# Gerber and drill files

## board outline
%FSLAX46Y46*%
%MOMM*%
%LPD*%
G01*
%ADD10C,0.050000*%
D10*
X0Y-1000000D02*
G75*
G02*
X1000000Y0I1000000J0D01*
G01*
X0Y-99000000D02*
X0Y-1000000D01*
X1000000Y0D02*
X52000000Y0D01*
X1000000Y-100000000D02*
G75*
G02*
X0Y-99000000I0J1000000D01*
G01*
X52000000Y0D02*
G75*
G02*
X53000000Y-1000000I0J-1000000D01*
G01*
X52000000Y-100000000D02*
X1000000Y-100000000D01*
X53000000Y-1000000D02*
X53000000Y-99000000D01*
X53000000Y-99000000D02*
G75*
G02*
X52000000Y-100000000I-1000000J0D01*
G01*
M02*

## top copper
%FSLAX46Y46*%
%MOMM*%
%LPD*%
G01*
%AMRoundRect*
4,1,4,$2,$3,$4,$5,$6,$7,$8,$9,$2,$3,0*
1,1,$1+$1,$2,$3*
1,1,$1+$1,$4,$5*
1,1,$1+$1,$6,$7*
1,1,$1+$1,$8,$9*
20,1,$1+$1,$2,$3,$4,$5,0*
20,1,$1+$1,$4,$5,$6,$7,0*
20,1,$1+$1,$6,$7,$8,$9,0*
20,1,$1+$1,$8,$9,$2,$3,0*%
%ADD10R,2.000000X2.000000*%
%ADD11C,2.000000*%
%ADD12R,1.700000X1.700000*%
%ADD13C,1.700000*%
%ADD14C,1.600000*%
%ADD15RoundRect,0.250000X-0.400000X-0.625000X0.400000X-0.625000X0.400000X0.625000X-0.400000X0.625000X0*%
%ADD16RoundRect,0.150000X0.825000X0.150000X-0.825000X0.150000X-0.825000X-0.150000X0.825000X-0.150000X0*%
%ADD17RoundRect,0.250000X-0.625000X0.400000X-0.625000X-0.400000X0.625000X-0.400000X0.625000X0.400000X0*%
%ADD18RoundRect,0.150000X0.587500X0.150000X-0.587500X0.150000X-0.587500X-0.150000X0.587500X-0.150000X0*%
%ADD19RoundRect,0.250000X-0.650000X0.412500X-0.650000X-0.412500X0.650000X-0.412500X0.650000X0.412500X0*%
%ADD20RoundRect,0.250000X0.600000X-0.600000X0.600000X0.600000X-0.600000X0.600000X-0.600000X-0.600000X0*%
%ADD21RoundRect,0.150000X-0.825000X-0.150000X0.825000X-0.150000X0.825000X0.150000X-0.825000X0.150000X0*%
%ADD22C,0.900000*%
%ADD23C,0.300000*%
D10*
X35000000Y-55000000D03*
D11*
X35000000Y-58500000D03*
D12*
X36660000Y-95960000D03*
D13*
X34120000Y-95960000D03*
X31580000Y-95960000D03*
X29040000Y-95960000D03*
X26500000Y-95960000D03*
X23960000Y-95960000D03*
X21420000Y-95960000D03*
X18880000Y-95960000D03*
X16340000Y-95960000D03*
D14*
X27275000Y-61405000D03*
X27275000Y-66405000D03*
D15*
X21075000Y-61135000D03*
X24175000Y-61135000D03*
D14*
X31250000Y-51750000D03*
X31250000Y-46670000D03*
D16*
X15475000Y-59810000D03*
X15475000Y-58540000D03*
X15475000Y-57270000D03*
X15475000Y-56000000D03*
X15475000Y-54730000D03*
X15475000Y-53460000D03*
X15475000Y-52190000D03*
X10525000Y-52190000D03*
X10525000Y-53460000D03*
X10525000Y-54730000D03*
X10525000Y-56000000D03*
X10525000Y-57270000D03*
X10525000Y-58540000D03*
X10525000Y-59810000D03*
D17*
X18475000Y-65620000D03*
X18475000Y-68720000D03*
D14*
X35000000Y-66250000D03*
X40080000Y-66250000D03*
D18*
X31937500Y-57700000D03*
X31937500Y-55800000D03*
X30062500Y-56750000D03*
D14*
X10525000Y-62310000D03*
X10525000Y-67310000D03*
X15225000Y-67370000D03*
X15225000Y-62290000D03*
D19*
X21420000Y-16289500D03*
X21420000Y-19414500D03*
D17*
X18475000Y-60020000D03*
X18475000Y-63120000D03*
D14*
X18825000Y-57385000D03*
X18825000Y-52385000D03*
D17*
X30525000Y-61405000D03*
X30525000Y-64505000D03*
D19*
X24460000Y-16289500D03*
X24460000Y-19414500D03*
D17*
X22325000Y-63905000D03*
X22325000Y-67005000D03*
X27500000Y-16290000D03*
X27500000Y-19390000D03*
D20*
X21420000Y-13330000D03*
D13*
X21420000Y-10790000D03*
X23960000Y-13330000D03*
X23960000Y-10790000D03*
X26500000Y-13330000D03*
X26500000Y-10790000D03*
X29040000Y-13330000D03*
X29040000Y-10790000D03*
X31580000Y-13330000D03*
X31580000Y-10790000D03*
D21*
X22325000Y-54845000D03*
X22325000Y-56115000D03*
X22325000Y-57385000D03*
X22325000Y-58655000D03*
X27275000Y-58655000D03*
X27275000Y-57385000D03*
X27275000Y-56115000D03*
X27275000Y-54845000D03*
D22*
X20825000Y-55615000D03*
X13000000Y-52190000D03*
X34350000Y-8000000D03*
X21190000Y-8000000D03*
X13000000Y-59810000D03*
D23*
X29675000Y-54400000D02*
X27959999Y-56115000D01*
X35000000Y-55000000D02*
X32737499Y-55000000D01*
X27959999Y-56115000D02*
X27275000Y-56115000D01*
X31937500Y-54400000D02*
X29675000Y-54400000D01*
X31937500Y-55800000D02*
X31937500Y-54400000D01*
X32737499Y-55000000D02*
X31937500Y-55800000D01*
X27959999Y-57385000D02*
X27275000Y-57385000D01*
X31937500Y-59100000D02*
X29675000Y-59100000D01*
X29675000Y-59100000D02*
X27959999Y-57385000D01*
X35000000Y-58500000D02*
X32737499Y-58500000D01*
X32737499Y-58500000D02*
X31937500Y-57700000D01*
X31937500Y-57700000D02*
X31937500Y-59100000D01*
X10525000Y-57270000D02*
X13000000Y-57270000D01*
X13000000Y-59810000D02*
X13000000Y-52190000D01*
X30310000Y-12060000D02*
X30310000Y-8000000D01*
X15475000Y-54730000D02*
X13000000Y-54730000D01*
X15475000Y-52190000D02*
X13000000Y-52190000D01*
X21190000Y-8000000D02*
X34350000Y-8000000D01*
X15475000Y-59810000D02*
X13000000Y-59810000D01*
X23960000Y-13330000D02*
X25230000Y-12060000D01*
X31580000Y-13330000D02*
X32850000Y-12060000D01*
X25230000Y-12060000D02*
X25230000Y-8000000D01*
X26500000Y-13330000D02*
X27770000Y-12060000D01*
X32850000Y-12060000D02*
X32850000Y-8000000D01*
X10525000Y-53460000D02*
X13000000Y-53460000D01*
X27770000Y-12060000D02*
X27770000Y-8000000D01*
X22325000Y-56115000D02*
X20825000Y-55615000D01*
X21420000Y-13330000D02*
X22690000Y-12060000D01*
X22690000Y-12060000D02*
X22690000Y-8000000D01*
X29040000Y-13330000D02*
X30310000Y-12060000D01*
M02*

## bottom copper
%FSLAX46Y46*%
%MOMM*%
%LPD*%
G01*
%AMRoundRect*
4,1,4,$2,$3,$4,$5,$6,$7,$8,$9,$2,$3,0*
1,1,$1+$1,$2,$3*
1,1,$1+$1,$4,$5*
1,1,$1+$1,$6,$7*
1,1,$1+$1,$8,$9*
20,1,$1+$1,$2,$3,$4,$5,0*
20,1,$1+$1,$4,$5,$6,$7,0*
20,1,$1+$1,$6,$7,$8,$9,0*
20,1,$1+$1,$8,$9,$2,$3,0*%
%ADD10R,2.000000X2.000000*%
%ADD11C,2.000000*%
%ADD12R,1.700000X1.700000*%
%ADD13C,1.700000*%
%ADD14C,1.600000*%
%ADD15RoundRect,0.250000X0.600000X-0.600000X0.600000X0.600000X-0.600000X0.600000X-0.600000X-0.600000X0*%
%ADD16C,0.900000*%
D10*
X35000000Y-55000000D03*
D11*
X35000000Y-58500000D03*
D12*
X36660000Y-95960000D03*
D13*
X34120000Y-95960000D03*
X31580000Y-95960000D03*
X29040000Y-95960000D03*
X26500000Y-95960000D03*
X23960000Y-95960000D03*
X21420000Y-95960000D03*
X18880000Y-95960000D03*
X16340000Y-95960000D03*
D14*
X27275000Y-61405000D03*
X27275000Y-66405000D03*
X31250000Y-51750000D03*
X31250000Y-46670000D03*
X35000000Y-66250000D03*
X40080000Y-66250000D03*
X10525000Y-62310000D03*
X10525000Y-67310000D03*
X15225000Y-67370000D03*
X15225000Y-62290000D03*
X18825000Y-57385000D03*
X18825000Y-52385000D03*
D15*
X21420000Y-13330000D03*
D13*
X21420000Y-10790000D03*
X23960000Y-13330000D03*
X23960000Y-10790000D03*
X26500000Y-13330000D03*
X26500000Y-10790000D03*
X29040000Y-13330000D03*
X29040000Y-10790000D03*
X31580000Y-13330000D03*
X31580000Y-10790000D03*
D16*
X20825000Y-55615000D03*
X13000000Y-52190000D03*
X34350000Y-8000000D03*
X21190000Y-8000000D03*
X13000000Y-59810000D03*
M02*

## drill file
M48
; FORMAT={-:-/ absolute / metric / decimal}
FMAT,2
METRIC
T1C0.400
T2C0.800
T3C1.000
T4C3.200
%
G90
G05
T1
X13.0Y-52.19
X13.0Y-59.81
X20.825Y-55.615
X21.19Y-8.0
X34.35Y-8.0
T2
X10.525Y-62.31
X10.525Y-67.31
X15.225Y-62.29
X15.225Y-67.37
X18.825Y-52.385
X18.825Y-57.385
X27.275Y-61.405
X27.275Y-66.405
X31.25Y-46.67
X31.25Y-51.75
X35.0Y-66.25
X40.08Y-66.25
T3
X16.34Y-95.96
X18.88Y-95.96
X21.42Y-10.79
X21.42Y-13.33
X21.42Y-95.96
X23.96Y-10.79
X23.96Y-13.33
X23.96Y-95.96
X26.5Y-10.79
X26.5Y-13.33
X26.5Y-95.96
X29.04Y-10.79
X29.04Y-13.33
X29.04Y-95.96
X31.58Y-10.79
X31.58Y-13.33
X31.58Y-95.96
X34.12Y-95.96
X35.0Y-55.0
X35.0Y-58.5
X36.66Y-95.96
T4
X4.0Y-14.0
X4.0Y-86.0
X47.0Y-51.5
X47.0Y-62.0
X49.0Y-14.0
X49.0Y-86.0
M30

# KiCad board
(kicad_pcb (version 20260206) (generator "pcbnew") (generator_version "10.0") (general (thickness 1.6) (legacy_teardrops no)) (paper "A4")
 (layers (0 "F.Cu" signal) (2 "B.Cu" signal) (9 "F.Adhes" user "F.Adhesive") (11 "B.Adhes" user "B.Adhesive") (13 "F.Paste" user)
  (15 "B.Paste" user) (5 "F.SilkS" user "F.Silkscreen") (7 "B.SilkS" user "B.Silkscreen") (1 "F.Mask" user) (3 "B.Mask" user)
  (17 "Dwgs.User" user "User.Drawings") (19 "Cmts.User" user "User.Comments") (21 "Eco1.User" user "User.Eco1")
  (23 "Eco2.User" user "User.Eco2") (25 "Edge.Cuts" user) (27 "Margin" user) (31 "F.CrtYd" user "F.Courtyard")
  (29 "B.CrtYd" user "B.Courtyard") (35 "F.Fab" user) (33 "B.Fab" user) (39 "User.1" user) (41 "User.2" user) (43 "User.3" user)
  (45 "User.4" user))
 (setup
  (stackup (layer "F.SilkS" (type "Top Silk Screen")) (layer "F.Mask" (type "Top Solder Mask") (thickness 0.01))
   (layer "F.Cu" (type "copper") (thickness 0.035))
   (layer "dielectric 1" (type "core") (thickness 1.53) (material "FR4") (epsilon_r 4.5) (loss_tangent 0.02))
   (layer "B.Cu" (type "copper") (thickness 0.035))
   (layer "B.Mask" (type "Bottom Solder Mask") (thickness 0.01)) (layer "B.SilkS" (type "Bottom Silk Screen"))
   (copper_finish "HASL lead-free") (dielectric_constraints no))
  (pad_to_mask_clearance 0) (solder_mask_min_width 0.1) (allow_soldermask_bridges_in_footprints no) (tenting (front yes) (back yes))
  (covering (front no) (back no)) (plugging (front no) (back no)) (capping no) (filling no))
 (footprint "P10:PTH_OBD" (layer "F.Cu") (at 35 55 -90)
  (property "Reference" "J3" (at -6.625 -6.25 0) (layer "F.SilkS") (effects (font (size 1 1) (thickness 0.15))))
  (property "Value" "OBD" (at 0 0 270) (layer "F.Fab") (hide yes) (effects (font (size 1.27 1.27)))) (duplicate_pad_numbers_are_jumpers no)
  (pad "" np_thru_hole circle (at -3.5 -12 270) (size 3.2 3.2) (drill 3.2) (layers "*.Cu" "*.Mask"))
  (pad "" np_thru_hole circle (at 7 -12 270) (size 3.2 3.2) (drill 3.2) (layers "*.Cu" "*.Mask"))
  (pad "1" thru_hole rect (at 0 0 270) (size 2 2) (drill 1) (layers "*.Cu" "*.Mask") (remove_unused_layers no) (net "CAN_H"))
  (pad "2" thru_hole circle (at 3.5 0 270) (size 2 2) (drill 1) (layers "*.Cu" "*.Mask") (remove_unused_layers no) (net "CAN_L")))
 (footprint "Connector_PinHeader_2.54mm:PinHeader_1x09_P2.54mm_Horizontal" (layer "F.Cu") (at 36.66 95.96 -90)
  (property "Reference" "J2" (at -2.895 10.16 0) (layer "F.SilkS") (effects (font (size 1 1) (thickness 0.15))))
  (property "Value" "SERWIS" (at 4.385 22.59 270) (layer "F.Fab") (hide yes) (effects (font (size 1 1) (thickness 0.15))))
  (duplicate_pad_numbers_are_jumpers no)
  (pad "1" thru_hole rect (at 0 0 270) (size 1.7 1.7) (drill 1) (layers "*.Cu" "*.Mask") (remove_unused_layers no) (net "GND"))
  (pad "2" thru_hole circle (at 0 2.54 270) (size 1.7 1.7) (drill 1) (layers "*.Cu" "*.Mask") (remove_unused_layers no)
   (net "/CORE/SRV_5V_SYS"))
  (pad "3" thru_hole circle (at 0 5.08 270) (size 1.7 1.7) (drill 1) (layers "*.Cu" "*.Mask") (remove_unused_layers no)
   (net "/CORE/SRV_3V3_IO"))
  (pad "4" thru_hole circle (at 0 7.62 270) (size 1.7 1.7) (drill 1) (layers "*.Cu" "*.Mask") (remove_unused_layers no)
   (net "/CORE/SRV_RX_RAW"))
  (pad "5" thru_hole circle (at 0 10.16 270) (size 1.7 1.7) (drill 1) (layers "*.Cu" "*.Mask") (remove_unused_layers no)
   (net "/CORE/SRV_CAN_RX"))
  (pad "6" thru_hole circle (at 0 12.7 270) (size 1.7 1.7) (drill 1) (layers "*.Cu" "*.Mask") (remove_unused_layers no)
   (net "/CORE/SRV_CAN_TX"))
  (pad "7" thru_hole circle (at 0 15.24 270) (size 1.7 1.7) (drill 1) (layers "*.Cu" "*.Mask") (remove_unused_layers no)
   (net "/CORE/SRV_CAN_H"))
  (pad "8" thru_hole circle (at 0 17.78 270) (size 1.7 1.7) (drill 1) (layers "*.Cu" "*.Mask") (remove_unused_layers no)
   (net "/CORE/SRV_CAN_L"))
  (pad "9" thru_hole circle (at 0 20.32 270) (size 1.7 1.7) (drill 1) (layers "*.Cu" "*.Mask") (remove_unused_layers no) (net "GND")))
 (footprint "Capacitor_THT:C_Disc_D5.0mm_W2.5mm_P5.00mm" (layer "F.Cu") (at 27.275 61.405 -90)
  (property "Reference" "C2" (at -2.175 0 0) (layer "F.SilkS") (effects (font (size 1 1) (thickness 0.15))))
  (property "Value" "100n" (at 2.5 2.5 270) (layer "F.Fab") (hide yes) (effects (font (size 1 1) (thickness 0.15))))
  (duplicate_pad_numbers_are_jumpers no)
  (pad "1" thru_hole circle (at 0 0 270) (size 1.6 1.6) (drill 0.8) (layers "*.Cu" "*.Mask") (remove_unused_layers no) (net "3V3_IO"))
  (pad "2" thru_hole circle (at 5 0 270) (size 1.6 1.6) (drill 0.8) (layers "*.Cu" "*.Mask") (remove_unused_layers no) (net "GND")))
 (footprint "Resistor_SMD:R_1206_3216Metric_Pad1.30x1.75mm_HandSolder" (layer "F.Cu") (at 22.625 61.135)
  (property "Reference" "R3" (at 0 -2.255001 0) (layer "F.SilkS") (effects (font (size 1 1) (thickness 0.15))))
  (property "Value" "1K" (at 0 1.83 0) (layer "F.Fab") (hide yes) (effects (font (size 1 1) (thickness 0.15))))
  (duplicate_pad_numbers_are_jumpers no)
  (pad "1" smd roundrect (at -1.55 0) (size 1.3 1.75) (layers "F.Cu" "F.Mask" "F.Paste") (roundrect_rratio 0.192308) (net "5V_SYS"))
  (pad "2" smd roundrect (at 1.55 0) (size 1.3 1.75) (layers "F.Cu" "F.Mask" "F.Paste") (roundrect_rratio 0.192308) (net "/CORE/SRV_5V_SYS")))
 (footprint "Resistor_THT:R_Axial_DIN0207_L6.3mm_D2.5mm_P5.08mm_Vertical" (layer "F.Cu") (at 31.25 51.75 90)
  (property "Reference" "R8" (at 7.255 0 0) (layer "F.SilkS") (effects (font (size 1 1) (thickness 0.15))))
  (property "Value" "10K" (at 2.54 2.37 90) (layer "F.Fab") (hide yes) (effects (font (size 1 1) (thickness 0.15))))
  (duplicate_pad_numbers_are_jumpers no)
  (pad "1" thru_hole circle (at 0 0 90) (size 1.6 1.6) (drill 0.8) (layers "*.Cu" "*.Mask") (remove_unused_layers no) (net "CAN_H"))
  (pad "2" thru_hole circle (at 5.08 0 90) (size 1.6 1.6) (drill 0.8) (layers "*.Cu" "*.Mask") (remove_unused_layers no)
   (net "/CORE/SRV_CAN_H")))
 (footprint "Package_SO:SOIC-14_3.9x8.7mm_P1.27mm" (layer "F.Cu") (at 13 56 180)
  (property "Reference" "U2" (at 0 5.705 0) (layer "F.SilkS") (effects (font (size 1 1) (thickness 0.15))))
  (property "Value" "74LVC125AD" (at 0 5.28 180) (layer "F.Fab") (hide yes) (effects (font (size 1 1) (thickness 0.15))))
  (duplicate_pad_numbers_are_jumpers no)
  (pad "1" smd roundrect (at -2.475 -3.81 180) (size 1.95 0.6) (layers "F.Cu" "F.Mask" "F.Paste") (roundrect_rratio 0.25) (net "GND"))
  (pad "2" smd roundrect (at -2.475 -2.54 180) (size 1.95 0.6) (layers "F.Cu" "F.Mask" "F.Paste") (roundrect_rratio 0.25) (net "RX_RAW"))
  (pad "3" smd roundrect (at -2.475 -1.27 180) (size 1.95 0.6) (layers "F.Cu" "F.Mask" "F.Paste") (roundrect_rratio 0.25)
   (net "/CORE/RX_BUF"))
  (pad "4" smd roundrect (at -2.475 0 180) (size 1.95 0.6) (layers "F.Cu" "F.Mask" "F.Paste") (roundrect_rratio 0.25) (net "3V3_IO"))
  (pad "5" smd roundrect (at -2.475 1.27 180) (size 1.95 0.6) (layers "F.Cu" "F.Mask" "F.Paste") (roundrect_rratio 0.25) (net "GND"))
  (pad "6" smd roundrect (at -2.475 2.54 180) (size 1.95 0.6) (layers "F.Cu" "F.Mask" "F.Paste") (roundrect_rratio 0.25)
   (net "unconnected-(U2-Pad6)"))
  (pad "7" smd roundrect (at -2.475 3.81 180) (size 1.95 0.6) (layers "F.Cu" "F.Mask" "F.Paste") (roundrect_rratio 0.25) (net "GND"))
  (pad "8" smd roundrect (at 2.475 3.81 180) (size 1.95 0.6) (layers "F.Cu" "F.Mask" "F.Paste") (roundrect_rratio 0.25)
   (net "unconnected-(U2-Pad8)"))
  (pad "9" smd roundrect (at 2.475 2.54 180) (size 1.95 0.6) (layers "F.Cu" "F.Mask" "F.Paste") (roundrect_rratio 0.25) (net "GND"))
  (pad "10" smd roundrect (at 2.475 1.27 180) (size 1.95 0.6) (layers "F.Cu" "F.Mask" "F.Paste") (roundrect_rratio 0.25) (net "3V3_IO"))
  (pad "11" smd roundrect (at 2.475 0 180) (size 1.95 0.6) (layers "F.Cu" "F.Mask" "F.Paste") (roundrect_rratio 0.25)
   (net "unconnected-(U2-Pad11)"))
  (pad "12" smd roundrect (at 2.475 -1.27 180) (size 1.95 0.6) (layers "F.Cu" "F.Mask" "F.Paste") (roundrect_rratio 0.25) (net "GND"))
  (pad "13" smd roundrect (at 2.475 -2.54 180) (size 1.95 0.6) (layers "F.Cu" "F.Mask" "F.Paste") (roundrect_rratio 0.25) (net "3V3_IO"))
  (pad "14" smd roundrect (at 2.475 -3.81 180) (size 1.95 0.6) (layers "F.Cu" "F.Mask" "F.Paste") (roundrect_rratio 0.25) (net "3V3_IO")))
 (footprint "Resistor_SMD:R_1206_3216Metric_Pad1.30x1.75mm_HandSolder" (layer "F.Cu") (at 18.475 67.17 -90)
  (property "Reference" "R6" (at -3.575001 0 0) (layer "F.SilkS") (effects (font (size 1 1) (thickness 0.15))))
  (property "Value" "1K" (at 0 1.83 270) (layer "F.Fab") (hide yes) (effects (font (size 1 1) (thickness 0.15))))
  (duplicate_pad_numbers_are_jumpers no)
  (pad "1" smd roundrect (at -1.55 0 270) (size 1.3 1.75) (layers "F.Cu" "F.Mask" "F.Paste") (roundrect_rratio 0.192308)
   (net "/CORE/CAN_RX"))
  (pad "2" smd roundrect (at 1.55 0 270) (size 1.3 1.75) (layers "F.Cu" "F.Mask" "F.Paste") (roundrect_rratio 0.192308)
   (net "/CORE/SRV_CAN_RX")))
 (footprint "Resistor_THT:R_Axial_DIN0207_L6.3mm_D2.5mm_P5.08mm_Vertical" (layer "F.Cu") (at 35 66.25)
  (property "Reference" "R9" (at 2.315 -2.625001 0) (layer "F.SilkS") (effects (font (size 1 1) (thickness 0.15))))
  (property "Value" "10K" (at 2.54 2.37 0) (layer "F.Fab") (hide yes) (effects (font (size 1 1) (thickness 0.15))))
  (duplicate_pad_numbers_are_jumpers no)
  (pad "1" thru_hole circle (at 0 0) (size 1.6 1.6) (drill 0.8) (layers "*.Cu" "*.Mask") (remove_unused_layers no) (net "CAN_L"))
  (pad "2" thru_hole circle (at 5.08 0) (size 1.6 1.6) (drill 0.8) (layers "*.Cu" "*.Mask") (remove_unused_layers no)
   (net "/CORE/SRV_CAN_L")))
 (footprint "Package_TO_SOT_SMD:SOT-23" (layer "F.Cu") (at 31 56.75 180)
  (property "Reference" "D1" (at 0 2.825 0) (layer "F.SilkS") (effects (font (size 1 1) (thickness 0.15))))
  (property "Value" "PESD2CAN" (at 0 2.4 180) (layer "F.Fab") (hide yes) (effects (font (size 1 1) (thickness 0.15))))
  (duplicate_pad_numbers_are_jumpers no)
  (pad "1" smd roundrect (at -0.9375 -0.95 180) (size 1.475 0.6) (layers "F.Cu" "F.Mask" "F.Paste") (roundrect_rratio 0.25) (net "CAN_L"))
  (pad "2" smd roundrect (at -0.9375 0.95 180) (size 1.475 0.6) (layers "F.Cu" "F.Mask" "F.Paste") (roundrect_rratio 0.25) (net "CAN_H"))
  (pad "3" smd roundrect (at 0.9375 0 180) (size 1.475 0.6) (layers "F.Cu" "F.Mask" "F.Paste") (roundrect_rratio 0.25) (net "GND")))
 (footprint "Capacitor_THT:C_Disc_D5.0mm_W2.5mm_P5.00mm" (layer "F.Cu") (at 10.525 62.31 -90)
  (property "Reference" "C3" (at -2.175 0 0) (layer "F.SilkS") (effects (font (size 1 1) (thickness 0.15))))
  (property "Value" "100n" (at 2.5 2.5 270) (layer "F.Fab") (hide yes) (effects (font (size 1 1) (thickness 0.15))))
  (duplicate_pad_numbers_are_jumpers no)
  (pad "1" thru_hole circle (at 0 0 270) (size 1.6 1.6) (drill 0.8) (layers "*.Cu" "*.Mask") (remove_unused_layers no) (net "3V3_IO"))
  (pad "2" thru_hole circle (at 5 0 270) (size 1.6 1.6) (drill 0.8) (layers "*.Cu" "*.Mask") (remove_unused_layers no) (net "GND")))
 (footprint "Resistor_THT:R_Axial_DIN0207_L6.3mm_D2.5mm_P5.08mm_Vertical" (layer "F.Cu") (at 15.225 67.37 90)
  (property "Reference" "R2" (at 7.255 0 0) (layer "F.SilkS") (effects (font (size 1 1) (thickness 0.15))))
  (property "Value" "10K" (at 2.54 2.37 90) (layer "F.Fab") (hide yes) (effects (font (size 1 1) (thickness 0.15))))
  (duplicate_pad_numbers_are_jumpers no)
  (pad "1" thru_hole circle (at 0 0 90) (size 1.6 1.6) (drill 0.8) (layers "*.Cu" "*.Mask") (remove_unused_layers no) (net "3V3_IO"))
  (pad "2" thru_hole circle (at 5.08 0 90) (size 1.6 1.6) (drill 0.8) (layers "*.Cu" "*.Mask") (remove_unused_layers no) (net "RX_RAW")))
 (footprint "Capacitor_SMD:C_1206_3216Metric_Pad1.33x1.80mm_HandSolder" (layer "F.Cu") (at 21.42 17.852 -90)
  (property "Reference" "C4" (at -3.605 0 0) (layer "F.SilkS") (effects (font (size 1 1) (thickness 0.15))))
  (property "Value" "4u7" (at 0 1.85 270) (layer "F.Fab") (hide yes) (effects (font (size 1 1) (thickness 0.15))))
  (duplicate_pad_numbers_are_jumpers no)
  (pad "1" smd roundrect (at -1.5625 0 270) (size 1.325 1.8) (layers "F.Cu" "F.Mask" "F.Paste") (roundrect_rratio 0.188679) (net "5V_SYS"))
  (pad "2" smd roundrect (at 1.5625 0 270) (size 1.325 1.8) (layers "F.Cu" "F.Mask" "F.Paste") (roundrect_rratio 0.188679) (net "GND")))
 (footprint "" (layer "F.Cu") (at 49 86)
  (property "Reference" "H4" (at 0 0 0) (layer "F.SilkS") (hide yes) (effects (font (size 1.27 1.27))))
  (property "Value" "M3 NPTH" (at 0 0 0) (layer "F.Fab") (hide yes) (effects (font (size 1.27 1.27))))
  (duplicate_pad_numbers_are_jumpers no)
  (pad "" np_thru_hole circle (at 0 0) (size 3.2 3.2) (drill 3.2) (layers "*.Cu")))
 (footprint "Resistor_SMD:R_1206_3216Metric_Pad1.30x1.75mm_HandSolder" (layer "F.Cu") (at 18.475 61.57 -90)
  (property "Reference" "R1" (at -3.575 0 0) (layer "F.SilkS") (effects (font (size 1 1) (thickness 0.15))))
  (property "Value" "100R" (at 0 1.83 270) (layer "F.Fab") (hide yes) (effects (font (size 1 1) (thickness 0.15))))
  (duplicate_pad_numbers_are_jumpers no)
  (pad "1" smd roundrect (at -1.55 0 270) (size 1.3 1.75) (layers "F.Cu" "F.Mask" "F.Paste") (roundrect_rratio 0.192308)
   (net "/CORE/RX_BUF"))
  (pad "2" smd roundrect (at 1.55 0 270) (size 1.3 1.75) (layers "F.Cu" "F.Mask" "F.Paste") (roundrect_rratio 0.192308) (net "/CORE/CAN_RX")))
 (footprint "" (layer "F.Cu") (at 49 14)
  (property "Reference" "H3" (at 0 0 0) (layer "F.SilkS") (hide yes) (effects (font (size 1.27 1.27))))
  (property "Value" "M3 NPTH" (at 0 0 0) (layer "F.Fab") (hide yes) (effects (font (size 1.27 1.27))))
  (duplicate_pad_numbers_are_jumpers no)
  (pad "" np_thru_hole circle (at 0 0) (size 3.2 3.2) (drill 3.2) (layers "*.Cu")))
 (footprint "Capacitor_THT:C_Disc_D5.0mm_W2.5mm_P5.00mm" (layer "F.Cu") (at 18.825 57.385 90)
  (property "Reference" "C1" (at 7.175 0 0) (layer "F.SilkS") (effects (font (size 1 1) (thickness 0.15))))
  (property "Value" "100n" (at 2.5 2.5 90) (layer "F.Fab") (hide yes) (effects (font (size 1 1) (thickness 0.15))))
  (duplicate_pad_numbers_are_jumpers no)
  (pad "1" thru_hole circle (at 0 0 90) (size 1.6 1.6) (drill 0.8) (layers "*.Cu" "*.Mask") (remove_unused_layers no) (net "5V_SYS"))
  (pad "2" thru_hole circle (at 5 0 90) (size 1.6 1.6) (drill 0.8) (layers "*.Cu" "*.Mask") (remove_unused_layers no) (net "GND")))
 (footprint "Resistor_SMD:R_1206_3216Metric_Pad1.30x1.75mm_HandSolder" (layer "F.Cu") (at 30.525 62.955 -90)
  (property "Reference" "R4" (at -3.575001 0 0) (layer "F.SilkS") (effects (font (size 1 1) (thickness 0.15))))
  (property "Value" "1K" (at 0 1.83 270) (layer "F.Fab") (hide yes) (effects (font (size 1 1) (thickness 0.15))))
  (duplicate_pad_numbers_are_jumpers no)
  (pad "1" smd roundrect (at -1.55 0 270) (size 1.3 1.75) (layers "F.Cu" "F.Mask" "F.Paste") (roundrect_rratio 0.192308) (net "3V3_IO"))
  (pad "2" smd roundrect (at 1.55 0 270) (size 1.3 1.75) (layers "F.Cu" "F.Mask" "F.Paste") (roundrect_rratio 0.192308)
   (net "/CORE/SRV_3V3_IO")))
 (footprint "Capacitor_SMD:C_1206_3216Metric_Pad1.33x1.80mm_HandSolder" (layer "F.Cu") (at 24.46 17.852 -90)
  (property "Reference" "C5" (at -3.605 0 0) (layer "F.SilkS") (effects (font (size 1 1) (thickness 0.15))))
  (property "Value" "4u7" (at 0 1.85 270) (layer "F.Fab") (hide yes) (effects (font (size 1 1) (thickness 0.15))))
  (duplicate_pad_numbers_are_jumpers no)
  (pad "1" smd roundrect (at -1.5625 0 270) (size 1.325 1.8) (layers "F.Cu" "F.Mask" "F.Paste") (roundrect_rratio 0.188679) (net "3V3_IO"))
  (pad "2" smd roundrect (at 1.5625 0 270) (size 1.325 1.8) (layers "F.Cu" "F.Mask" "F.Paste") (roundrect_rratio 0.188679) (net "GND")))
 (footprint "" (layer "F.Cu") (at 4 86)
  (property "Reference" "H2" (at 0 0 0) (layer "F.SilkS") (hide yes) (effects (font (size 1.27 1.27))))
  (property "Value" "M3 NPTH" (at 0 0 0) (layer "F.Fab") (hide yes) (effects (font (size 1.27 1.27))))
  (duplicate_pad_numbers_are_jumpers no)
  (pad "" np_thru_hole circle (at 0 0) (size 3.2 3.2) (drill 3.2) (layers "*.Cu")))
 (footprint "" (layer "F.Cu") (at 4 14)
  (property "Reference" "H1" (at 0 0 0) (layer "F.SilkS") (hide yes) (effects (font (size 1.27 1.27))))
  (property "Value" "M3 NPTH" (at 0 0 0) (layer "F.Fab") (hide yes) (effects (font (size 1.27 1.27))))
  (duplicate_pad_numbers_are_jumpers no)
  (pad "" np_thru_hole circle (at 0 0) (size 3.2 3.2) (drill 3.2) (layers "*.Cu")))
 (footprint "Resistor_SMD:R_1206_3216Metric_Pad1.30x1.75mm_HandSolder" (layer "F.Cu") (at 22.325 65.455 -90)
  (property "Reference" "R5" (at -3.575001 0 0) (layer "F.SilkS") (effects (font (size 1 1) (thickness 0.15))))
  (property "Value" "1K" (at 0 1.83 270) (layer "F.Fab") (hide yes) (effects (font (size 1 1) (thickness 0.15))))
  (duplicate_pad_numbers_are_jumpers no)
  (pad "1" smd roundrect (at -1.55 0 270) (size 1.3 1.75) (layers "F.Cu" "F.Mask" "F.Paste") (roundrect_rratio 0.192308) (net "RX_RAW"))
  (pad "2" smd roundrect (at 1.55 0 270) (size 1.3 1.75) (layers "F.Cu" "F.Mask" "F.Paste") (roundrect_rratio 0.192308)
   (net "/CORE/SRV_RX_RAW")))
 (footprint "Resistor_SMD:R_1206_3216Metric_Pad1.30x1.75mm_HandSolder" (layer "F.Cu") (at 27.5 17.84 -90)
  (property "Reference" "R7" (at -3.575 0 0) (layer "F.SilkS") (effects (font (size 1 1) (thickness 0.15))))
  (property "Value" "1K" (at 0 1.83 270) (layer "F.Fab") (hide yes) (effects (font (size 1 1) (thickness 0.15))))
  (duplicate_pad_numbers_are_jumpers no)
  (pad "1" smd roundrect (at -1.55 0 270) (size 1.3 1.75) (layers "F.Cu" "F.Mask" "F.Paste") (roundrect_rratio 0.192308)
   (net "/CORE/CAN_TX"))
  (pad "2" smd roundrect (at 1.55 0 270) (size 1.3 1.75) (layers "F.Cu" "F.Mask" "F.Paste") (roundrect_rratio 0.192308)
   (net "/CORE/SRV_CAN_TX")))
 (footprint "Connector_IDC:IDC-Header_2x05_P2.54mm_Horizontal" (layer "F.Cu") (at 21.42 13.33 90)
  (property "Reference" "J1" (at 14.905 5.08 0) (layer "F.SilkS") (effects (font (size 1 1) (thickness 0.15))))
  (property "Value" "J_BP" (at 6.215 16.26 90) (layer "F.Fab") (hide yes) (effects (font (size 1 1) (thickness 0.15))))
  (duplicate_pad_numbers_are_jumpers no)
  (pad "1" thru_hole roundrect (at 0 0 90) (size 1.7 1.7) (drill 1) (layers "*.Cu" "*.Mask") (remove_unused_layers no)
   (roundrect_rratio 0.147059) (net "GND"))
  (pad "2" thru_hole circle (at 2.54 0 90) (size 1.7 1.7) (drill 1) (layers "*.Cu" "*.Mask") (remove_unused_layers no) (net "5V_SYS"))
  (pad "3" thru_hole circle (at 0 2.54 90) (size 1.7 1.7) (drill 1) (layers "*.Cu" "*.Mask") (remove_unused_layers no) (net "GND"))
  (pad "4" thru_hole circle (at 2.54 2.54 90) (size 1.7 1.7) (drill 1) (layers "*.Cu" "*.Mask") (remove_unused_layers no) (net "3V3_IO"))
  (pad "5" thru_hole circle (at 0 5.08 90) (size 1.7 1.7) (drill 1) (layers "*.Cu" "*.Mask") (remove_unused_layers no) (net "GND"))
  (pad "6" thru_hole circle (at 2.54 5.08 90) (size 1.7 1.7) (drill 1) (layers "*.Cu" "*.Mask") (remove_unused_layers no)
   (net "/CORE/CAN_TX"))
  (pad "7" thru_hole circle (at 0 7.62 90) (size 1.7 1.7) (drill 1) (layers "*.Cu" "*.Mask") (remove_unused_layers no) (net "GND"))
  (pad "8" thru_hole circle (at 2.54 7.62 90) (size 1.7 1.7) (drill 1) (layers "*.Cu" "*.Mask") (remove_unused_layers no)
   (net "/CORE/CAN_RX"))
  (pad "9" thru_hole circle (at 0 10.16 90) (size 1.7 1.7) (drill 1) (layers "*.Cu" "*.Mask") (remove_unused_layers no) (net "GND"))
  (pad "10" thru_hole circle (at 2.54 10.16 90) (size 1.7 1.7) (drill 1) (layers "*.Cu" "*.Mask") (remove_unused_layers no) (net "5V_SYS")))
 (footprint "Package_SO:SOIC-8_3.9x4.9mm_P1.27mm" (layer "F.Cu") (at 24.8 56.75)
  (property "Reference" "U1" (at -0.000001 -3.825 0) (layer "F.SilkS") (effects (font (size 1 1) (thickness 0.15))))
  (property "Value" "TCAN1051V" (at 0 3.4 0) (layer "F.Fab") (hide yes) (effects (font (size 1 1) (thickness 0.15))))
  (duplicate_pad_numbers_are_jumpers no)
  (pad "1" smd roundrect (at -2.475 -1.905) (size 1.95 0.6) (layers "F.Cu" "F.Mask" "F.Paste") (roundrect_rratio 0.25) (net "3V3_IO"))
  (pad "2" smd roundrect (at -2.475 -0.635) (size 1.95 0.6) (layers "F.Cu" "F.Mask" "F.Paste") (roundrect_rratio 0.25) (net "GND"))
  (pad "3" smd roundrect (at -2.475 0.635) (size 1.95 0.6) (layers "F.Cu" "F.Mask" "F.Paste") (roundrect_rratio 0.25) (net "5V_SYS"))
  (pad "4" smd roundrect (at -2.475 1.905) (size 1.95 0.6) (layers "F.Cu" "F.Mask" "F.Paste") (roundrect_rratio 0.25) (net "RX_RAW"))
  (pad "5" smd roundrect (at 2.475 1.905) (size 1.95 0.6) (layers "F.Cu" "F.Mask" "F.Paste") (roundrect_rratio 0.25) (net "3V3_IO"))
  (pad "6" smd roundrect (at 2.475 0.635) (size 1.95 0.6) (layers "F.Cu" "F.Mask" "F.Paste") (roundrect_rratio 0.25) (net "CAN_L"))
  (pad "7" smd roundrect (at 2.475 -0.635) (size 1.95 0.6) (layers "F.Cu" "F.Mask" "F.Paste") (roundrect_rratio 0.25) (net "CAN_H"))
  (pad "8" smd roundrect (at 2.475 -1.905) (size 1.95 0.6) (layers "F.Cu" "F.Mask" "F.Paste") (roundrect_rratio 0.25) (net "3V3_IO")))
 (gr_arc (start 0 1) (mid 0.292893 0.292893) (end 1 0) (stroke (width 0.05) (type default)) (layer "Edge.Cuts"))
 (gr_line (start 0 99) (end 0 1) (stroke (width 0.05) (type default)) (layer "Edge.Cuts"))
 (gr_line (start 1 0) (end 52 0) (stroke (width 0.05) (type default)) (layer "Edge.Cuts"))
 (gr_arc (start 1 100) (mid 0.292893 99.707107) (end 0 99) (stroke (width 0.05) (type default)) (layer "Edge.Cuts"))
 (gr_arc (start 52 0) (mid 52.707107 0.292893) (end 53 1) (stroke (width 0.05) (type default)) (layer "Edge.Cuts"))
 (gr_line (start 52 100) (end 1 100) (stroke (width 0.05) (type default)) (layer "Edge.Cuts"))
 (gr_line (start 53 1) (end 53 99) (stroke (width 0.05) (type default)) (layer "Edge.Cuts"))
 (gr_arc (start 53 99) (mid 52.707107 99.707107) (end 52 100) (stroke (width 0.05) (type default)) (layer "Edge.Cuts"))
 (segment (start 29.675 54.4) (end 27.959999 56.115) (width 0.3) (locked yes) (layer "F.Cu") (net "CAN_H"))
 (segment (start 35 55) (end 32.737499 55) (width 0.3) (locked yes) (layer "F.Cu") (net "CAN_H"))
 (segment (start 27.959999 56.115) (end 27.275 56.115) (width 0.3) (locked yes) (layer "F.Cu") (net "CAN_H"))
 (segment (start 31.9375 54.4) (end 29.675 54.4) (width 0.3) (locked yes) (layer "F.Cu") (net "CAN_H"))
 (segment (start 31.9375 55.8) (end 31.9375 54.4) (width 0.3) (locked yes) (layer "F.Cu") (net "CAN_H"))
 (segment (start 32.737499 55) (end 31.9375 55.8) (width 0.3) (locked yes) (layer "F.Cu") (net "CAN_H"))
 (segment (start 27.959999 57.385) (end 27.275 57.385) (width 0.3) (locked yes) (layer "F.Cu") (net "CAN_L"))
 (segment (start 31.9375 59.1) (end 29.675 59.1) (width 0.3) (locked yes) (layer "F.Cu") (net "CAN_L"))
 (segment (start 29.675 59.1) (end 27.959999 57.385) (width 0.3) (locked yes) (layer "F.Cu") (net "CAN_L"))
 (segment (start 35 58.5) (end 32.737499 58.5) (width 0.3) (locked yes) (layer "F.Cu") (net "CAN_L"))
 (segment (start 32.737499 58.5) (end 31.9375 57.7) (width 0.3) (locked yes) (layer "F.Cu") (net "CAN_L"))
 (segment (start 31.9375 57.7) (end 31.9375 59.1) (width 0.3) (locked yes) (layer "F.Cu") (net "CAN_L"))
 (segment (start 10.525 57.27) (end 13 57.27) (width 0.3) (locked yes) (layer "F.Cu") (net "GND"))
 (segment (start 13 59.81) (end 13 52.19) (width 0.3) (locked yes) (layer "F.Cu") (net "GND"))
 (segment (start 30.31 12.06) (end 30.31 8) (width 0.3) (locked yes) (layer "F.Cu") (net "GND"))
 (segment (start 15.475 54.73) (end 13 54.73) (width 0.3) (locked yes) (layer "F.Cu") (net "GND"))
 (segment (start 15.475 52.19) (end 13 52.19) (width 0.3) (locked yes) (layer "F.Cu") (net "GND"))
 (segment (start 21.19 8) (end 34.35 8) (width 0.3) (locked yes) (layer "F.Cu") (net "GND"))
 (segment (start 15.475 59.81) (end 13 59.81) (width 0.3) (locked yes) (layer "F.Cu") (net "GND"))
 (segment (start 23.96 13.33) (end 25.23 12.06) (width 0.3) (locked yes) (layer "F.Cu") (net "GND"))
 (segment (start 31.58 13.33) (end 32.85 12.06) (width 0.3) (locked yes) (layer "F.Cu") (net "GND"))
 (segment (start 25.23 12.06) (end 25.23 8) (width 0.3) (locked yes) (layer "F.Cu") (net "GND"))
 (segment (start 26.5 13.33) (end 27.77 12.06) (width 0.3) (locked yes) (layer "F.Cu") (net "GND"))
 (segment (start 32.85 12.06) (end 32.85 8) (width 0.3) (locked yes) (layer "F.Cu") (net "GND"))
 (segment (start 10.525 53.46) (end 13 53.46) (width 0.3) (locked yes) (layer "F.Cu") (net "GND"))
 (segment (start 27.77 12.06) (end 27.77 8) (width 0.3) (locked yes) (layer "F.Cu") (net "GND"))
 (segment (start 22.325 56.115) (end 20.825 55.615) (width 0.3) (locked yes) (layer "F.Cu") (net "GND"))
 (segment (start 21.42 13.33) (end 22.69 12.06) (width 0.3) (locked yes) (layer "F.Cu") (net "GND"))
 (segment (start 22.69 12.06) (end 22.69 8) (width 0.3) (locked yes) (layer "F.Cu") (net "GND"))
 (segment (start 29.04 13.33) (end 30.31 12.06) (width 0.3) (locked yes) (layer "F.Cu") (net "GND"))
 (via (at 20.825 55.615) (size 0.9) (drill 0.4) (layers "F.Cu" "B.Cu") (locked yes) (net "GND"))
 (via (at 13 52.19) (size 0.9) (drill 0.4) (layers "F.Cu" "B.Cu") (locked yes) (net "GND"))
 (via (at 34.35 8) (size 0.9) (drill 0.4) (layers "F.Cu" "B.Cu") (locked yes) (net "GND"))
 (via (at 21.19 8) (size 0.9) (drill 0.4) (layers "F.Cu" "B.Cu") (locked yes) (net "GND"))
 (via (at 13 59.81) (size 0.9) (drill 0.4) (layers "F.Cu" "B.Cu") (locked yes) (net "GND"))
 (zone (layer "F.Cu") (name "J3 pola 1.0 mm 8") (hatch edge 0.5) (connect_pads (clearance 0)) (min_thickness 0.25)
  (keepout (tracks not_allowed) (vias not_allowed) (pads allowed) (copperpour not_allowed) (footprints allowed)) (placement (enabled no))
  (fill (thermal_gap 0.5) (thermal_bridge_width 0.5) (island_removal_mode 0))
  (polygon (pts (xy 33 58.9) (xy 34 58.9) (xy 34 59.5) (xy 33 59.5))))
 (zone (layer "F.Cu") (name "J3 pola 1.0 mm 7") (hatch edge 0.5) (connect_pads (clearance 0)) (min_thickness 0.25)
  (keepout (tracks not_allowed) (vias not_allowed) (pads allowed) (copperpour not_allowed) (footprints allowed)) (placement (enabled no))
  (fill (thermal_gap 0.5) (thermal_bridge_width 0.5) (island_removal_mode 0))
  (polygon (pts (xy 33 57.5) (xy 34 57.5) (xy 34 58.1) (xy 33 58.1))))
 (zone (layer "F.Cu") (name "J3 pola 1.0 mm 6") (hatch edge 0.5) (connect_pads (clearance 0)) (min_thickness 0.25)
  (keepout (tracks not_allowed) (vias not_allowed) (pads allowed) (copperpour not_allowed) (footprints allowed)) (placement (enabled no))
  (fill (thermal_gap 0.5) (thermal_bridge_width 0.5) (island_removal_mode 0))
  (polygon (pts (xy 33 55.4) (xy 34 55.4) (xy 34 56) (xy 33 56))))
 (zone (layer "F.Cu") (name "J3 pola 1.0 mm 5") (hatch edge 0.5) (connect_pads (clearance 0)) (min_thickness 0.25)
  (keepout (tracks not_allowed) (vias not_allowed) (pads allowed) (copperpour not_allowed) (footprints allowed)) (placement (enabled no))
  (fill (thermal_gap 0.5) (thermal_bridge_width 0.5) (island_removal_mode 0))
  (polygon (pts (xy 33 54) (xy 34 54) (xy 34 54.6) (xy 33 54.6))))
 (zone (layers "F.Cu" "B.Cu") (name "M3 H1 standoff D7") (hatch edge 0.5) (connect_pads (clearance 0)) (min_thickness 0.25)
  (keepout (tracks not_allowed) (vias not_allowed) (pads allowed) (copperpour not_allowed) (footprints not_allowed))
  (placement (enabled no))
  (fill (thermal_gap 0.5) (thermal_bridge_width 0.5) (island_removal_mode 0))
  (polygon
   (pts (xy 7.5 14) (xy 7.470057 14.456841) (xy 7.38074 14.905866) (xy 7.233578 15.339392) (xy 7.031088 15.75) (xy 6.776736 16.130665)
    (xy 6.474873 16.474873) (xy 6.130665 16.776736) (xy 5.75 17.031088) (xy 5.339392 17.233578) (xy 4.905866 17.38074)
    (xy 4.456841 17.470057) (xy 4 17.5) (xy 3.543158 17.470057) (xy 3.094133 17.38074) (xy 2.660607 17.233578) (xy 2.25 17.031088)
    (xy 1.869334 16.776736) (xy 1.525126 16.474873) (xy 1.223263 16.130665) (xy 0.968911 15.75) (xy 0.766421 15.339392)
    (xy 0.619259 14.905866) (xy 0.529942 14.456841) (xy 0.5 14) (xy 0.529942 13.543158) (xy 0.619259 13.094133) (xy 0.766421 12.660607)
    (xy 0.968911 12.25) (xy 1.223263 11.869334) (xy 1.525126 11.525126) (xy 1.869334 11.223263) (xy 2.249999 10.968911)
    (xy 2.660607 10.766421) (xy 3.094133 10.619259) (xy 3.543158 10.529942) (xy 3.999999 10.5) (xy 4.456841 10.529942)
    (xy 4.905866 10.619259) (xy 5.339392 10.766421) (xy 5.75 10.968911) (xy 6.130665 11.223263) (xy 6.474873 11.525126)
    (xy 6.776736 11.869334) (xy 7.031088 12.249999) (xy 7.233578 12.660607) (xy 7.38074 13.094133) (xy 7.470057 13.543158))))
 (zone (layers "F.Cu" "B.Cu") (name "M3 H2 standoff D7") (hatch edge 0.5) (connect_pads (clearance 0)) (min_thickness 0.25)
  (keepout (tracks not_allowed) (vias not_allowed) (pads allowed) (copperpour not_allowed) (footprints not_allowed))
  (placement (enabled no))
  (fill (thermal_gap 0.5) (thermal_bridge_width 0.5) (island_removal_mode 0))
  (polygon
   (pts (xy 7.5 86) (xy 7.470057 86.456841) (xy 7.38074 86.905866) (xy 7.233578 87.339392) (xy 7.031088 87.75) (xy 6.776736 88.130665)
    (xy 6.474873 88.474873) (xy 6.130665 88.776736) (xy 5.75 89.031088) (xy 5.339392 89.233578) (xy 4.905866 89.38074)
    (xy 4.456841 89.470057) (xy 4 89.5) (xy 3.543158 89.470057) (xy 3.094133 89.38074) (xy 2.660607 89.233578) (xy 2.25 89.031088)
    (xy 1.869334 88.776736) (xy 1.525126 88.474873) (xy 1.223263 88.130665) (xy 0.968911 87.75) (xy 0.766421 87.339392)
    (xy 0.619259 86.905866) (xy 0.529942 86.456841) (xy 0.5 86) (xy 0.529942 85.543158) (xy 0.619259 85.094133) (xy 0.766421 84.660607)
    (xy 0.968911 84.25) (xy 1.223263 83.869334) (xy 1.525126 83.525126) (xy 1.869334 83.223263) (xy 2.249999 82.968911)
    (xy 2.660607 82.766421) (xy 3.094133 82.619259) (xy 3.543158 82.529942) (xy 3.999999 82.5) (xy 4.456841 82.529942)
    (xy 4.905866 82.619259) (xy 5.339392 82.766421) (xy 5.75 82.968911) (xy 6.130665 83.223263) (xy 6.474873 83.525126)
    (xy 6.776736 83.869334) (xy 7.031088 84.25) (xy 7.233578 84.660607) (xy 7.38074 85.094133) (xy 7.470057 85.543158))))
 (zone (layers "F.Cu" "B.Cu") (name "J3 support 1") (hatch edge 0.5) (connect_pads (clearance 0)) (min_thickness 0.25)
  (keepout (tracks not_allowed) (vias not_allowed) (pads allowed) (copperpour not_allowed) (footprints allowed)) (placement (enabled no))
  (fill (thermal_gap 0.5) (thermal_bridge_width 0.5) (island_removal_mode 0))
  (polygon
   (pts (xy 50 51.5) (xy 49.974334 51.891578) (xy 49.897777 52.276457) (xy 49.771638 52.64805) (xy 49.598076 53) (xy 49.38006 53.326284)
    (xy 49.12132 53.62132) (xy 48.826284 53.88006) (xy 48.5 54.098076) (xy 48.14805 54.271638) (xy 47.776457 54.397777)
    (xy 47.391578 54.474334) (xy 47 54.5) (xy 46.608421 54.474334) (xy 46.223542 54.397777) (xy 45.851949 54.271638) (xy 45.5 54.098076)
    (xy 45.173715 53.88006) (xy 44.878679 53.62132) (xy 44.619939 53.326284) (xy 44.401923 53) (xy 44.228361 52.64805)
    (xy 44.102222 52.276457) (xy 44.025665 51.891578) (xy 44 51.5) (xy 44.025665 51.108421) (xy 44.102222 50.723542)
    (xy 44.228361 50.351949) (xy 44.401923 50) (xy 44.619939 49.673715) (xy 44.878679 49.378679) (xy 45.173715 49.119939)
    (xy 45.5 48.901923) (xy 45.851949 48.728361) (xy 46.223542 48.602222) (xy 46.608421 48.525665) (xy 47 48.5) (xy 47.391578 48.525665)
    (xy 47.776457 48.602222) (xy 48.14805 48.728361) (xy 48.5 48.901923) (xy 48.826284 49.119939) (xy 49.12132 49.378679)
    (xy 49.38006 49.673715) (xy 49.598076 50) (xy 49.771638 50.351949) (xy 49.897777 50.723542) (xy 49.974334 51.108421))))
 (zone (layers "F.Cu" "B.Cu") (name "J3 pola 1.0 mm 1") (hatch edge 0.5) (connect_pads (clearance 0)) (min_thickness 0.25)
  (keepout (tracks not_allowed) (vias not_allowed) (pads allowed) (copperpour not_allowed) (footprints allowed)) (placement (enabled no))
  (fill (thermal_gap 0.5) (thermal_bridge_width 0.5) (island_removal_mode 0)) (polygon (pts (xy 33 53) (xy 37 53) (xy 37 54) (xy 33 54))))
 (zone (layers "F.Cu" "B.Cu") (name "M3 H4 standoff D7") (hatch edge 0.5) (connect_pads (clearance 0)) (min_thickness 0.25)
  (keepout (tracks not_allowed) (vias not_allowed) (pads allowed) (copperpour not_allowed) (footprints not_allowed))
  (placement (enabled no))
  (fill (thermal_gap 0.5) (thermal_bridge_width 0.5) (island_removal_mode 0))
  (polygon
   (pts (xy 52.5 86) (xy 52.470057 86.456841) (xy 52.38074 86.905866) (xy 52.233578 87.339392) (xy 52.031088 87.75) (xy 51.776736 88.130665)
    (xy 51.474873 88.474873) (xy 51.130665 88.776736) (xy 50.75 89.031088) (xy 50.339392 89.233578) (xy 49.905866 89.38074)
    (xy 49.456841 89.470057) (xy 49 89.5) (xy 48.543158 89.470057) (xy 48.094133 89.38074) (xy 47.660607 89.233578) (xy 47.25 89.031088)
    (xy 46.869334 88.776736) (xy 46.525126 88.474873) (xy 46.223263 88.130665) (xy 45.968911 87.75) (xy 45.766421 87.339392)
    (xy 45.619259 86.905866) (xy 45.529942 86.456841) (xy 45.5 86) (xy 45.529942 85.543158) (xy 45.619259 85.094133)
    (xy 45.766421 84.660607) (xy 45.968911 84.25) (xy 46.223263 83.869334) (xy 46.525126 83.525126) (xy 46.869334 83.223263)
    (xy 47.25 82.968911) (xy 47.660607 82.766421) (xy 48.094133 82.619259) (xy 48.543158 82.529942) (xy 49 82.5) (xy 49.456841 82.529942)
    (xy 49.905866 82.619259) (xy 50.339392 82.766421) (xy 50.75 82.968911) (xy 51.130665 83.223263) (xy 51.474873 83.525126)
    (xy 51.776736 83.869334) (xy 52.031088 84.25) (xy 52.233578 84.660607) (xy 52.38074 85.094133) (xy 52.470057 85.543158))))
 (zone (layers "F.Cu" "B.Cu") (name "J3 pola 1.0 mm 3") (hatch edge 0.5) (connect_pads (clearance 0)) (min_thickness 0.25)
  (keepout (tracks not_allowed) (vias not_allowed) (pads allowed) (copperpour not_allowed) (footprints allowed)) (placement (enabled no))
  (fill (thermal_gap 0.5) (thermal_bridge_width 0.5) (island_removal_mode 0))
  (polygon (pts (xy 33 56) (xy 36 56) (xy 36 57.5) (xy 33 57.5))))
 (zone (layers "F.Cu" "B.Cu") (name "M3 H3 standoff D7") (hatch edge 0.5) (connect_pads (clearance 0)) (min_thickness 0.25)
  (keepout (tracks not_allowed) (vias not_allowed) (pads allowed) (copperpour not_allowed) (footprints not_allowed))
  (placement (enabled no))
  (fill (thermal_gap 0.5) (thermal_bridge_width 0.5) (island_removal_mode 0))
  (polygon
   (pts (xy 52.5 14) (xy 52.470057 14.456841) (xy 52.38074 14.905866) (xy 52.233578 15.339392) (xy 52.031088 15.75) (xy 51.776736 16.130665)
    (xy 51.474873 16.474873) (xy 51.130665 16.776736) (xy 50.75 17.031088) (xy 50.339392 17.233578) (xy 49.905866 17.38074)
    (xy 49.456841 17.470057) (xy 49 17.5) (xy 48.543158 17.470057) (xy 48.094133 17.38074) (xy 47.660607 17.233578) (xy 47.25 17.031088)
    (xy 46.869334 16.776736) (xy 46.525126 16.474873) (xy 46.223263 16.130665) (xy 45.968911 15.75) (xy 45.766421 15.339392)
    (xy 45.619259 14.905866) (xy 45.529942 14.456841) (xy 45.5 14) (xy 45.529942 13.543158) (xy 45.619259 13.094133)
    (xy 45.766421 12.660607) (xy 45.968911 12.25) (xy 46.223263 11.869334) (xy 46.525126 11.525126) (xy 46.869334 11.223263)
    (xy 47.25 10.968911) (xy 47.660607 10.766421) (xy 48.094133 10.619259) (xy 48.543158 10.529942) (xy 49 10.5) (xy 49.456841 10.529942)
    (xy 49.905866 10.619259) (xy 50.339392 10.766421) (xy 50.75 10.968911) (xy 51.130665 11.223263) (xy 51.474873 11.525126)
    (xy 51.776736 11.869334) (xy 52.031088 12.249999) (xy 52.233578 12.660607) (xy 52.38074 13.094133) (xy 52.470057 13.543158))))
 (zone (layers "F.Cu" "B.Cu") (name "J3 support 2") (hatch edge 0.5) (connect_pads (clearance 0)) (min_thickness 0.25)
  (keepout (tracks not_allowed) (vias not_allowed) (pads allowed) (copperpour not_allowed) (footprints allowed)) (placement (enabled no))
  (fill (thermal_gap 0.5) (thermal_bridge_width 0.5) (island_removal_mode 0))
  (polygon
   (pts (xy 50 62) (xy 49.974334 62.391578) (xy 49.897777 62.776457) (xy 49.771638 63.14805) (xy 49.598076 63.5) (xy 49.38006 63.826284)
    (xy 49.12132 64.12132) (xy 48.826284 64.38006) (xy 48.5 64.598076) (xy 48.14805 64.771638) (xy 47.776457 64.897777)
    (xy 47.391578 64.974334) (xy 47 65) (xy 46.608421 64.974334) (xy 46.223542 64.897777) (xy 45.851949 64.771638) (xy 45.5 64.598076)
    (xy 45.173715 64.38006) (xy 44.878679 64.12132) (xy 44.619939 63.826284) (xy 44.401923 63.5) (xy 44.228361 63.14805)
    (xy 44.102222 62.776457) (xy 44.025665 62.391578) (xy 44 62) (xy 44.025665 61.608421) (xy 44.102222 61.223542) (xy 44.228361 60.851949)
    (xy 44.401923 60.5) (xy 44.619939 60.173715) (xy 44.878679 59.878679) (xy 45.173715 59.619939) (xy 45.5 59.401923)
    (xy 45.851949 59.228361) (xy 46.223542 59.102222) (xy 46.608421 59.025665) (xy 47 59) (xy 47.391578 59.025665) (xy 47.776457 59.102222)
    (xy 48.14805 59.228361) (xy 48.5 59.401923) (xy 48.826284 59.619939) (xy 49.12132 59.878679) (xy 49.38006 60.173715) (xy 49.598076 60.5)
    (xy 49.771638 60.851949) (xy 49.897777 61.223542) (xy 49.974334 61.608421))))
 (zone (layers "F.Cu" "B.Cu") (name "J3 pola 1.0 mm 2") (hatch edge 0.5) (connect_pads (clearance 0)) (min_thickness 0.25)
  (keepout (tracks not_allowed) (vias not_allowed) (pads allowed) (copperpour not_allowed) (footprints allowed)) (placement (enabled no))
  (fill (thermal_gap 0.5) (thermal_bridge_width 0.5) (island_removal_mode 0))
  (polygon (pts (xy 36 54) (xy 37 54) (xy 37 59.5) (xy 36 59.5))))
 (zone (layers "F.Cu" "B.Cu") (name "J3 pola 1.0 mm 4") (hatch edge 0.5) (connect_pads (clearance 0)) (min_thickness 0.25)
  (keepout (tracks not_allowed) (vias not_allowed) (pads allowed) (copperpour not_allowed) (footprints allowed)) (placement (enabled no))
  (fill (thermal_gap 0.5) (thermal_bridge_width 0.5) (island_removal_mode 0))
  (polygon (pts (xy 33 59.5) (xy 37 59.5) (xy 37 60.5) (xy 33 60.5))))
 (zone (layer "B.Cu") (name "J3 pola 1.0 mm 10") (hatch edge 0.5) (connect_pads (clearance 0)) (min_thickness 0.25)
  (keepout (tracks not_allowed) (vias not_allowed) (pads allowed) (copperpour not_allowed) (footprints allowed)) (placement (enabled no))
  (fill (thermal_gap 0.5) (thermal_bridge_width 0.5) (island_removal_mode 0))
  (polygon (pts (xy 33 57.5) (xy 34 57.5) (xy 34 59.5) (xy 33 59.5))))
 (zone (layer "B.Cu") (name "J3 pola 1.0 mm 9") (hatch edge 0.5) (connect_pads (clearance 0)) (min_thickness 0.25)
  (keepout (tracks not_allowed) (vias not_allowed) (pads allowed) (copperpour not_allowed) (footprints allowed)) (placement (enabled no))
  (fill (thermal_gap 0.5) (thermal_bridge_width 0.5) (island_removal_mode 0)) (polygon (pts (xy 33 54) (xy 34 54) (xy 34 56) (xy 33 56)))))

